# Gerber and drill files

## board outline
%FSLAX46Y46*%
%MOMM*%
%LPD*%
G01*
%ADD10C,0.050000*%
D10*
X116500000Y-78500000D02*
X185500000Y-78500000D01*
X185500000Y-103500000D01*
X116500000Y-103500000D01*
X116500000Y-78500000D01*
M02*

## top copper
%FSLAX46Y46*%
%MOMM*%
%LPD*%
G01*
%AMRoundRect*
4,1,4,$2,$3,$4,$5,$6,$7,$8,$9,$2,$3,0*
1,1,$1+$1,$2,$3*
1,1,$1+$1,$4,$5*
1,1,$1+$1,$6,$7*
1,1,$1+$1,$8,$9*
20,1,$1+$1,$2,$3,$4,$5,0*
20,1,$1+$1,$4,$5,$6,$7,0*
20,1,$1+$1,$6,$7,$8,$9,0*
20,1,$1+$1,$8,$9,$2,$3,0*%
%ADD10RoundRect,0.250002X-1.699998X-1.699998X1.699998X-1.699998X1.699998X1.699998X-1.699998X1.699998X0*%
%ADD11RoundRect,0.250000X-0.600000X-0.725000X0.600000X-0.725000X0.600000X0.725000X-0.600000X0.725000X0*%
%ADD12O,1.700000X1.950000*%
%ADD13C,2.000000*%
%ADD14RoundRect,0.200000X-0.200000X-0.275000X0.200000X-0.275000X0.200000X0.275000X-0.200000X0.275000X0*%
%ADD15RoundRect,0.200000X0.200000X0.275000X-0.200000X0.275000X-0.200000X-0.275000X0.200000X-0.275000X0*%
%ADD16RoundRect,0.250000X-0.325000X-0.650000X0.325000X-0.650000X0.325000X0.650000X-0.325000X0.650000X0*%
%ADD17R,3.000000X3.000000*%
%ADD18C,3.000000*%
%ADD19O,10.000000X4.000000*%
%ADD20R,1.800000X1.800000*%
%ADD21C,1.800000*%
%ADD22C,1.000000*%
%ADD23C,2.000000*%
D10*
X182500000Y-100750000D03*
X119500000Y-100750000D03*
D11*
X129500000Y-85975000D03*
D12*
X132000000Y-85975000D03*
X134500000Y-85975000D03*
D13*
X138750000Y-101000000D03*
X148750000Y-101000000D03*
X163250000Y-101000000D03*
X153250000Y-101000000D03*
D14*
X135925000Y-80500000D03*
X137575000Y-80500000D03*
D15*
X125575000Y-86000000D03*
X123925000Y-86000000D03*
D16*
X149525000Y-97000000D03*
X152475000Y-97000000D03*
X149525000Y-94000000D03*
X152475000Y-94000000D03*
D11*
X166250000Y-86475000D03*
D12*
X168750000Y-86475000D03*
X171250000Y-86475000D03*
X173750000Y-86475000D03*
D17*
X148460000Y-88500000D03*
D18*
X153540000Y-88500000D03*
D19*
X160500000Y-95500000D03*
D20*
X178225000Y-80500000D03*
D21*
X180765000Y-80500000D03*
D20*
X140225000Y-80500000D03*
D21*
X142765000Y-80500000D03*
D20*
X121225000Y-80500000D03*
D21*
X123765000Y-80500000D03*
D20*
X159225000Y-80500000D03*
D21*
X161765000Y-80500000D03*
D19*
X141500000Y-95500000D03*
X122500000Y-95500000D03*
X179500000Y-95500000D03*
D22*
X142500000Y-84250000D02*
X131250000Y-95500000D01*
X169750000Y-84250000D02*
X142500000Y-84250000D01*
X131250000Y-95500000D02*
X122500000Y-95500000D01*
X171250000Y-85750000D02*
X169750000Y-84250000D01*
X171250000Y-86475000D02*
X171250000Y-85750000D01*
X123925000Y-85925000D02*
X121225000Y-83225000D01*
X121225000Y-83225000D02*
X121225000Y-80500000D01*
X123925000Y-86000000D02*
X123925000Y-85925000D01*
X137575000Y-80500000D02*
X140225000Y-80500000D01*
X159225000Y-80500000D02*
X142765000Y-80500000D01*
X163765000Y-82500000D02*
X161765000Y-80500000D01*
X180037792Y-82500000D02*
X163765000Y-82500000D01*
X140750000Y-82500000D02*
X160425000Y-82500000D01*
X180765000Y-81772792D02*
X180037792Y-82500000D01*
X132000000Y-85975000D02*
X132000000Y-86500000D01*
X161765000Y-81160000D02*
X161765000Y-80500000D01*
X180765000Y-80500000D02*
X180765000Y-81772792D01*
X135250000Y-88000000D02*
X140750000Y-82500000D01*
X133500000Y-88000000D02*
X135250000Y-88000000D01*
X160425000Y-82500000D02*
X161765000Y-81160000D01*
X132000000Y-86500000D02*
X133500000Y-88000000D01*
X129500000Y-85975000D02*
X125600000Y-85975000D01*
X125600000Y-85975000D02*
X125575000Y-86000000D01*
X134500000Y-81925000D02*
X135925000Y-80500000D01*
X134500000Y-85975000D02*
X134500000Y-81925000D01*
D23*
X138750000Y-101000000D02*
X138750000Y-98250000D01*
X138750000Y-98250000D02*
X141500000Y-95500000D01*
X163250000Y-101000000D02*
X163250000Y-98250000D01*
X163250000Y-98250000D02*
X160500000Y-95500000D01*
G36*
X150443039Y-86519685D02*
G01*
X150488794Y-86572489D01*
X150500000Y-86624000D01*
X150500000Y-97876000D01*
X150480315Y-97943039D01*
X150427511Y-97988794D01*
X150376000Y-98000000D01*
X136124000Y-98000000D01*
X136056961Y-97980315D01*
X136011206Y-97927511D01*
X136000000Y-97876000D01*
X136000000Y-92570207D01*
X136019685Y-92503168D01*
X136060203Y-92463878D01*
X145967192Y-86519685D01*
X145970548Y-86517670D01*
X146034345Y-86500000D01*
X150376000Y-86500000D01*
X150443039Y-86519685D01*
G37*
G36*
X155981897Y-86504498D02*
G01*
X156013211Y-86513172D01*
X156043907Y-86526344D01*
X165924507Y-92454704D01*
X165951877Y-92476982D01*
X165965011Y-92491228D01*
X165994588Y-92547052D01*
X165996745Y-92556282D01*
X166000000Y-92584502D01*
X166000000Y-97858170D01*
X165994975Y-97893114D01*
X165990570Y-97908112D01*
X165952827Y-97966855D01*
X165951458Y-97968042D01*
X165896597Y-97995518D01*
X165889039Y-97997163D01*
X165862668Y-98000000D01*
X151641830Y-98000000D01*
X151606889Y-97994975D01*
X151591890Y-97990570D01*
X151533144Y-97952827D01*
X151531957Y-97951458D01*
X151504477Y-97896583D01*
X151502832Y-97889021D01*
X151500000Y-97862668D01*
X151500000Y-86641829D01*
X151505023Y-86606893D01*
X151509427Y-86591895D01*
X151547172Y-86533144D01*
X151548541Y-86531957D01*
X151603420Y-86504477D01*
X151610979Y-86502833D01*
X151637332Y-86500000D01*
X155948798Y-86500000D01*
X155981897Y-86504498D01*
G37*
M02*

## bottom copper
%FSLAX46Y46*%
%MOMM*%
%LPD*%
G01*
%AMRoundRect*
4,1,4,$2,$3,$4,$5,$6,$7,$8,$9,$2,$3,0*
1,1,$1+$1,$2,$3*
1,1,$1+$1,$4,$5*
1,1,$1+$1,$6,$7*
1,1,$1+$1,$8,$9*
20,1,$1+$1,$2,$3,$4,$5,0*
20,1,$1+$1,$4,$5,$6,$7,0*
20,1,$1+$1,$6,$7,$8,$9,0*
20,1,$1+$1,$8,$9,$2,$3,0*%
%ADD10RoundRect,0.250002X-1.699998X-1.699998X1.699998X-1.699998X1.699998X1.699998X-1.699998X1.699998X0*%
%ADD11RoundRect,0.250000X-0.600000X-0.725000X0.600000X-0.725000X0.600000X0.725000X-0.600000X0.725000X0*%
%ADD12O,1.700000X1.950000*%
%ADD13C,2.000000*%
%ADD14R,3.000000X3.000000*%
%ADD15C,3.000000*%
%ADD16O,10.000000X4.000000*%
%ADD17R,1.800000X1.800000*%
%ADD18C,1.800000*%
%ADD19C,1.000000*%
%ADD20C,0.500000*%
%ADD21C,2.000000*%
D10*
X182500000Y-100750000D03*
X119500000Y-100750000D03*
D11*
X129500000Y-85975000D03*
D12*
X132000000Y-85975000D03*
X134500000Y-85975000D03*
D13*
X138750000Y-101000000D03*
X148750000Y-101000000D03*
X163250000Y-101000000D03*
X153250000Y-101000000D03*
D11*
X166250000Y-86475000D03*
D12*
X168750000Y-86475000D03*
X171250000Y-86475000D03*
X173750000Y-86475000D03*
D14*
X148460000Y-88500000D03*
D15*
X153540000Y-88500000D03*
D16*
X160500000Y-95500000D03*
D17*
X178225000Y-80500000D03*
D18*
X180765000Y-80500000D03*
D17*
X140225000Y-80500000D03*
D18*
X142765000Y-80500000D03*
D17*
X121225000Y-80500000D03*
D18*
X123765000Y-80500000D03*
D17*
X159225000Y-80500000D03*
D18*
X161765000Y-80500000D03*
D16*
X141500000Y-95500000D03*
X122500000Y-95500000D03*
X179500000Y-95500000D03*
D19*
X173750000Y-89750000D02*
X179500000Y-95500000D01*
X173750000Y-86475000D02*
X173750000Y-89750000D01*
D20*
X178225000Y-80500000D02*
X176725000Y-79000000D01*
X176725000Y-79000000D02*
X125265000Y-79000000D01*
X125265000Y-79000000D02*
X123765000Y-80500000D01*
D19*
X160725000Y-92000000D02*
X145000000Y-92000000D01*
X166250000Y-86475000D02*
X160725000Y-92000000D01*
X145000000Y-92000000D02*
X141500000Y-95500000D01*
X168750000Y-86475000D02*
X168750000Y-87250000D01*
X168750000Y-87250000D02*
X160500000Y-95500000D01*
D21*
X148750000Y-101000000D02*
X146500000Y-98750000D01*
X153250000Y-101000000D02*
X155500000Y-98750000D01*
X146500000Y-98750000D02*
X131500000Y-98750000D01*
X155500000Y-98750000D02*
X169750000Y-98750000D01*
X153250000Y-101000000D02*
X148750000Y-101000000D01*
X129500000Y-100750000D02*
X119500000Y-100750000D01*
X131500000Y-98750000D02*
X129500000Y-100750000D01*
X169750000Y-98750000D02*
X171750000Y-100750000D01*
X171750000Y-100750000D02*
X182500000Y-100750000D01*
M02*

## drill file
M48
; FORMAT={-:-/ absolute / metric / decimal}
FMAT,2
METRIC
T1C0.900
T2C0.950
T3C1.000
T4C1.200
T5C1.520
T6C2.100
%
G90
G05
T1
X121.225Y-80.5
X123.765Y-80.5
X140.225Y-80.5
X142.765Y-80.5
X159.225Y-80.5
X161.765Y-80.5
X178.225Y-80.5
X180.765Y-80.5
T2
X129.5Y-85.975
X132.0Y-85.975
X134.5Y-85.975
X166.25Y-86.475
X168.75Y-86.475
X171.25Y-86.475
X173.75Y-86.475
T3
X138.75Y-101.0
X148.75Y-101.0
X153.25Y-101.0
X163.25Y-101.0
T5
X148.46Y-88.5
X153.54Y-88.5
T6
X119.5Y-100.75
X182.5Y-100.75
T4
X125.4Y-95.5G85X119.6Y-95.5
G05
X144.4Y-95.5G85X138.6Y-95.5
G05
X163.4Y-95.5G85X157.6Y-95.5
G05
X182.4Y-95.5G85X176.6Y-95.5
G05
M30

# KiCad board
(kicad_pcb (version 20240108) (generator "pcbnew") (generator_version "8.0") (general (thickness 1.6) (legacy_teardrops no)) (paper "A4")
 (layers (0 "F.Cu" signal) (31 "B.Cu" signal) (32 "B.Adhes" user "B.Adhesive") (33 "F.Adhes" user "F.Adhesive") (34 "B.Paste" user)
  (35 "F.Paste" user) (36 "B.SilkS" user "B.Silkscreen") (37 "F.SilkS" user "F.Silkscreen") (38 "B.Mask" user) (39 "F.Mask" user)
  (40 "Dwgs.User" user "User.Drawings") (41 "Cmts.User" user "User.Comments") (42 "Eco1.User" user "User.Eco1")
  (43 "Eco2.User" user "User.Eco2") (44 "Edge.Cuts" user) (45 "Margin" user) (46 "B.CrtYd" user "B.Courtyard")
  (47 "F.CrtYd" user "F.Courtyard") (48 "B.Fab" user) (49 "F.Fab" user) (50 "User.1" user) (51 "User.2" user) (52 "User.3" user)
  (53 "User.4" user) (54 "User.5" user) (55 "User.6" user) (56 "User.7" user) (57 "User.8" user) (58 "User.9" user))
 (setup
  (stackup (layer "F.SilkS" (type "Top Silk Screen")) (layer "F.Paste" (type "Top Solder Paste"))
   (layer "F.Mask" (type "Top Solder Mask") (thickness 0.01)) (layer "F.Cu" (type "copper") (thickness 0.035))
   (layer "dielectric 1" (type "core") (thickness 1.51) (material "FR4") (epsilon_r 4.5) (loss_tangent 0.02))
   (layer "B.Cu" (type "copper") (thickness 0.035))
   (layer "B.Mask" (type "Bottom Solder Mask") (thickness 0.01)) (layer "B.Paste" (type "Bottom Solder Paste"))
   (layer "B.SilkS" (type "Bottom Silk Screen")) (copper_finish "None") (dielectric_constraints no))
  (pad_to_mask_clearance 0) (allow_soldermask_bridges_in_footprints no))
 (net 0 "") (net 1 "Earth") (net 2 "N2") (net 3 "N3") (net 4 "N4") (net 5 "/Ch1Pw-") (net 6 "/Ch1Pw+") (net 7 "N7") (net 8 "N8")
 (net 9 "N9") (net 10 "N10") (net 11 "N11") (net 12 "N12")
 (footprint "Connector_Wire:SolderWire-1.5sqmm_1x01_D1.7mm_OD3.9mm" (layer "F.Cu") (at 182.5 100.75)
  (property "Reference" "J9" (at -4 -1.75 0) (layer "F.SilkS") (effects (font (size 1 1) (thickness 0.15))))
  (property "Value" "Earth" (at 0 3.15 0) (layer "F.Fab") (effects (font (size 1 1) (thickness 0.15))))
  (pad "1" thru_hole roundrect (at 0 0) (size 3.9 3.9) (drill 2.1) (layers "*.Cu" "*.Mask") (remove_unused_layers no)
   (roundrect_rratio 0.064103) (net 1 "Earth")))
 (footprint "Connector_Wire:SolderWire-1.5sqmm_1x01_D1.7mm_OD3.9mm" (layer "F.Cu") (at 119.5 100.75)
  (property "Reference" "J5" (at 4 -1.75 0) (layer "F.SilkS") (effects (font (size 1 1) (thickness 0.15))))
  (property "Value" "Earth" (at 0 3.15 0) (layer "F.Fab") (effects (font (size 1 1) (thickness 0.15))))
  (pad "1" thru_hole roundrect (at 0 0) (size 3.9 3.9) (drill 2.1) (layers "*.Cu" "*.Mask") (remove_unused_layers no)
   (roundrect_rratio 0.064103) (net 1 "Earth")))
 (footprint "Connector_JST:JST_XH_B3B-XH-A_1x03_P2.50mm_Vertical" (layer "F.Cu") (at 129.5 85.975)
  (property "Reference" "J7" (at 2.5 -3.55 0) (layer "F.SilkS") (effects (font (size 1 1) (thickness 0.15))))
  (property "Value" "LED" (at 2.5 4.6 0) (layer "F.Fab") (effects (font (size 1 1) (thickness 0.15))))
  (pad "1" thru_hole roundrect (at 0 0) (size 1.7 1.95) (drill 0.95) (layers "*.Cu" "*.Mask") (remove_unused_layers no)
   (roundrect_rratio 0.147059) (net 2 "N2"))
  (pad "2" thru_hole oval (at 2.5 0) (size 1.7 1.95) (drill 0.95) (layers "*.Cu" "*.Mask") (remove_unused_layers no) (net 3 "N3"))
  (pad "3" thru_hole oval (at 5 0) (size 1.7 1.95) (drill 0.95) (layers "*.Cu" "*.Mask") (remove_unused_layers no) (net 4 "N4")))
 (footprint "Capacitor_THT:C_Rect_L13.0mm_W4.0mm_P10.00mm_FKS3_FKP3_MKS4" (layer "F.Cu") (at 138.75 101)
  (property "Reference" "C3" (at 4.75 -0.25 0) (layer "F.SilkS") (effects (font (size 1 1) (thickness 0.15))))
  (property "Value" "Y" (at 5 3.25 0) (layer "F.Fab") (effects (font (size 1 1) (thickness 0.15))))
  (pad "1" thru_hole circle (at 0 0) (size 2 2) (drill 1) (layers "*.Cu" "*.Mask") (remove_unused_layers no) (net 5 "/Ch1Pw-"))
  (pad "2" thru_hole circle (at 10 0) (size 2 2) (drill 1) (layers "*.Cu" "*.Mask") (remove_unused_layers no) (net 1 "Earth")))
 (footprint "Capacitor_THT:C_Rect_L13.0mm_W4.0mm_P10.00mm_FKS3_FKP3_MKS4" (layer "F.Cu") (at 163.25 101 180)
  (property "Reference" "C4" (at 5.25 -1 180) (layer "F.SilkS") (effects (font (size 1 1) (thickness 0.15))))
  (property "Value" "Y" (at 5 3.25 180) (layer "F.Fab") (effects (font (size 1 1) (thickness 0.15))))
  (pad "1" thru_hole circle (at 0 0 180) (size 2 2) (drill 1) (layers "*.Cu" "*.Mask") (remove_unused_layers no) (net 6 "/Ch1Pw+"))
  (pad "2" thru_hole circle (at 10 0 180) (size 2 2) (drill 1) (layers "*.Cu" "*.Mask") (remove_unused_layers no) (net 1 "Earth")))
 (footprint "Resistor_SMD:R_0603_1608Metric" (layer "F.Cu") (at 136.75 80.5)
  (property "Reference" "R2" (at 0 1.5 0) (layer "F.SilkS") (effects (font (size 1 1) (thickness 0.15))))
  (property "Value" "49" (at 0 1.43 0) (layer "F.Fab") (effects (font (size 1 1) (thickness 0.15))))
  (pad "1" smd roundrect (at -0.825 0) (size 0.8 0.95) (layers "F.Cu" "F.Paste" "F.Mask") (roundrect_rratio 0.25) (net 4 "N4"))
  (pad "2" smd roundrect (at 0.825 0) (size 0.8 0.95) (layers "F.Cu" "F.Paste" "F.Mask") (roundrect_rratio 0.25) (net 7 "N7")))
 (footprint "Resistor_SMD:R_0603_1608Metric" (layer "F.Cu") (at 124.75 86 180)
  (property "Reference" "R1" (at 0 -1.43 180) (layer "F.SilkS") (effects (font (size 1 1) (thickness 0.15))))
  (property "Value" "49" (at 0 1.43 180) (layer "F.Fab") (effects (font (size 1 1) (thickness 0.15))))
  (pad "1" smd roundrect (at -0.825 0 180) (size 0.8 0.95) (layers "F.Cu" "F.Paste" "F.Mask") (roundrect_rratio 0.25) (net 2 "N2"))
  (pad "2" smd roundrect (at 0.825 0 180) (size 0.8 0.95) (layers "F.Cu" "F.Paste" "F.Mask") (roundrect_rratio 0.25) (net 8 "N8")))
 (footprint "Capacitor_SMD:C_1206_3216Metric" (layer "F.Cu") (at 151 97)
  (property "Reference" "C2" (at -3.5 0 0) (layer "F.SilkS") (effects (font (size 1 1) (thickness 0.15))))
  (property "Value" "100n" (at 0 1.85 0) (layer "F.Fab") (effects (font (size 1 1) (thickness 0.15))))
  (pad "1" smd roundrect (at -1.475 0) (size 1.15 1.8) (layers "F.Cu" "F.Paste" "F.Mask") (roundrect_rratio 0.217391) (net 5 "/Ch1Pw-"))
  (pad "2" smd roundrect (at 1.475 0) (size 1.15 1.8) (layers "F.Cu" "F.Paste" "F.Mask") (roundrect_rratio 0.217391) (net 6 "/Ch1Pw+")))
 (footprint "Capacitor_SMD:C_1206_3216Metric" (layer "F.Cu") (at 151 94)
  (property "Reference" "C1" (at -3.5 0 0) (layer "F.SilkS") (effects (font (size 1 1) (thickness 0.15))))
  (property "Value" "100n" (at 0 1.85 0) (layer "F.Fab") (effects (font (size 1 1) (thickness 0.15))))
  (pad "1" smd roundrect (at -1.475 0) (size 1.15 1.8) (layers "F.Cu" "F.Paste" "F.Mask") (roundrect_rratio 0.217391) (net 5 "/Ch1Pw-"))
  (pad "2" smd roundrect (at 1.475 0) (size 1.15 1.8) (layers "F.Cu" "F.Paste" "F.Mask") (roundrect_rratio 0.217391) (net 6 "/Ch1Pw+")))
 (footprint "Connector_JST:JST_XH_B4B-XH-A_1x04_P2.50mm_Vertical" (layer "F.Cu") (at 166.25 86.475)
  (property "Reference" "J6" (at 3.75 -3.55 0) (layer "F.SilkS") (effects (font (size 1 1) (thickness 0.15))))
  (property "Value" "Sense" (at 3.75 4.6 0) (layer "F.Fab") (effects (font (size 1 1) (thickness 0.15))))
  (pad "1" thru_hole roundrect (at 0 0) (size 1.7 1.95) (drill 0.95) (layers "*.Cu" "*.Mask") (remove_unused_layers no)
   (roundrect_rratio 0.147059) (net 5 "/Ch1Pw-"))
  (pad "2" thru_hole oval (at 2.5 0) (size 1.7 1.95) (drill 0.95) (layers "*.Cu" "*.Mask") (remove_unused_layers no) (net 6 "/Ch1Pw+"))
  (pad "3" thru_hole oval (at 5 0) (size 1.7 1.95) (drill 0.95) (layers "*.Cu" "*.Mask") (remove_unused_layers no) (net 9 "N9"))
  (pad "4" thru_hole oval (at 7.5 0) (size 1.7 1.95) (drill 0.95) (layers "*.Cu" "*.Mask") (remove_unused_layers no) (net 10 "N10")))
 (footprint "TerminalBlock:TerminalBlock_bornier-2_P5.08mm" (layer "F.Cu") (at 148.46 88.5)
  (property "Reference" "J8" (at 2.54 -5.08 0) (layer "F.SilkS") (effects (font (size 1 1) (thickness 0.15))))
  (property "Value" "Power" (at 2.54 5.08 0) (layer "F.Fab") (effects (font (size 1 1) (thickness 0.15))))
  (pad "1" thru_hole rect (at 0 0) (size 3 3) (drill 1.52) (layers "*.Cu" "*.Mask") (remove_unused_layers no) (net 5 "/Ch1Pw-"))
  (pad "2" thru_hole circle (at 5.08 0) (size 3 3) (drill 1.52) (layers "*.Cu" "*.Mask") (remove_unused_layers no) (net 6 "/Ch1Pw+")))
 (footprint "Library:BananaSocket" (layer "B.Cu") (at 160.5 95.5 180)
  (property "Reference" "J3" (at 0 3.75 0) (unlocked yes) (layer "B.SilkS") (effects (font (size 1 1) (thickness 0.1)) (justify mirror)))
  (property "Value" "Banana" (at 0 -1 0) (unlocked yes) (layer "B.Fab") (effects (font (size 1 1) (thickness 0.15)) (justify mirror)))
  (pad "1" thru_hole oval (at 0 0 180) (size 10 4) (drill oval 7 1.2) (layers "*.Cu" "*.Mask") (remove_unused_layers no) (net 6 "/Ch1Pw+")))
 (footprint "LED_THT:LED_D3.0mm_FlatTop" (layer "B.Cu") (at 178.225 80.5)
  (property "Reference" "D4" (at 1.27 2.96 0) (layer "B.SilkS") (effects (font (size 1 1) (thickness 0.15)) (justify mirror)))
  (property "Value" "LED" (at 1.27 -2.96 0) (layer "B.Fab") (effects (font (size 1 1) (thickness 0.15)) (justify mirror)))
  (pad "1" thru_hole rect (at 0 0) (size 1.8 1.8) (drill 0.9) (layers "*.Cu" "*.Mask") (remove_unused_layers no) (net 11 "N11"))
  (pad "2" thru_hole circle (at 2.54 0) (size 1.8 1.8) (drill 0.9) (layers "*.Cu" "*.Mask") (remove_unused_layers no) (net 3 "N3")))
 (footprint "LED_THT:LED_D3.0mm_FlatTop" (layer "B.Cu") (at 140.225 80.5)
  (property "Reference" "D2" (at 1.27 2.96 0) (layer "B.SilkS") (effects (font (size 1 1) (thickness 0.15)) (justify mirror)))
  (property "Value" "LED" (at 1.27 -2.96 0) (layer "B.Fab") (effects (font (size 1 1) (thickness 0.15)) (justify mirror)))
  (pad "1" thru_hole rect (at 0 0) (size 1.8 1.8) (drill 0.9) (layers "*.Cu" "*.Mask") (remove_unused_layers no) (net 7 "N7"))
  (pad "2" thru_hole circle (at 2.54 0) (size 1.8 1.8) (drill 0.9) (layers "*.Cu" "*.Mask") (remove_unused_layers no) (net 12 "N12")))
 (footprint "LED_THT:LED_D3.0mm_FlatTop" (layer "B.Cu") (at 121.225 80.5)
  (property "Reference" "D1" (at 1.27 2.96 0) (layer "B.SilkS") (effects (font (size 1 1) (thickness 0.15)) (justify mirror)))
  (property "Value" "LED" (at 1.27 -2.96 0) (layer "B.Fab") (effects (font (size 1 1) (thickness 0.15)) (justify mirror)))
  (pad "1" thru_hole rect (at 0 0) (size 1.8 1.8) (drill 0.9) (layers "*.Cu" "*.Mask") (remove_unused_layers no) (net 8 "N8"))
  (pad "2" thru_hole circle (at 2.54 0) (size 1.8 1.8) (drill 0.9) (layers "*.Cu" "*.Mask") (remove_unused_layers no) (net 11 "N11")))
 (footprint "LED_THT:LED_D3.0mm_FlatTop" (layer "B.Cu") (at 159.225 80.5)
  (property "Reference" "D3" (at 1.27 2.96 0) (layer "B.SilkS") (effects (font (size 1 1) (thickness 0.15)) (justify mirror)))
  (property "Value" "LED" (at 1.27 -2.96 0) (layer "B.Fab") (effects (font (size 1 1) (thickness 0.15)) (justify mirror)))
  (pad "1" thru_hole rect (at 0 0) (size 1.8 1.8) (drill 0.9) (layers "*.Cu" "*.Mask") (remove_unused_layers no) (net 12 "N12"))
  (pad "2" thru_hole circle (at 2.54 0) (size 1.8 1.8) (drill 0.9) (layers "*.Cu" "*.Mask") (remove_unused_layers no) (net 3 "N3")))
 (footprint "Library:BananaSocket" (layer "B.Cu") (at 141.5 95.5 180)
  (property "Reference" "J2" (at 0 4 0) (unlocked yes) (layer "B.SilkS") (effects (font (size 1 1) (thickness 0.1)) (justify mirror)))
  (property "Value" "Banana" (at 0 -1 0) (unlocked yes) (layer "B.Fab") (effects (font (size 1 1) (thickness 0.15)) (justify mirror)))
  (pad "1" thru_hole oval (at 0 0 180) (size 10 4) (drill oval 7 1.2) (layers "*.Cu" "*.Mask") (remove_unused_layers no) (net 5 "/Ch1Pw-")))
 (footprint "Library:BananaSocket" (layer "B.Cu") (at 122.5 95.5 180)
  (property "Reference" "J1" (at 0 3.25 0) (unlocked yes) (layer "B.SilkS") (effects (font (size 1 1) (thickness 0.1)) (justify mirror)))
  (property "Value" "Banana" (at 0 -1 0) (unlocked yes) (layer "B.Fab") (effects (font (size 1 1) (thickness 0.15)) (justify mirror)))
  (pad "1" thru_hole oval (at 0 0 180) (size 10 4) (drill oval 7 1.2) (layers "*.Cu" "*.Mask") (remove_unused_layers no) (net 9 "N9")))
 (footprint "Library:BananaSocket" (layer "B.Cu") (at 179.5 95.5 180)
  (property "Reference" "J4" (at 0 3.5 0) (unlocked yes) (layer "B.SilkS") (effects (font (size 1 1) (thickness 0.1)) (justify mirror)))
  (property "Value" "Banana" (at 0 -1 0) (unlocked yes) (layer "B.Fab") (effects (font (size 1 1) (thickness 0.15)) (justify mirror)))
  (pad "1" thru_hole oval (at 0 0 180) (size 10 4) (drill oval 7 1.2) (layers "*.Cu" "*.Mask") (remove_unused_layers no) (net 10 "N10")))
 (gr_rect (start 116.5 78.5) (end 185.5 103.5) (stroke (width 0.05) (type default)) (fill none) (layer "Edge.Cuts"))
 (segment (start 142.5 84.25) (end 131.25 95.5) (width 1) (layer "F.Cu") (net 9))
 (segment (start 169.75 84.25) (end 142.5 84.25) (width 1) (layer "F.Cu") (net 9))
 (segment (start 131.25 95.5) (end 122.5 95.5) (width 1) (layer "F.Cu") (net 9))
 (segment (start 171.25 85.75) (end 169.75 84.25) (width 1) (layer "F.Cu") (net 9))
 (segment (start 171.25 86.475) (end 171.25 85.75) (width 1) (layer "F.Cu") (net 9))
 (segment (start 173.75 89.75) (end 179.5 95.5) (width 1) (layer "B.Cu") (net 10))
 (segment (start 173.75 86.475) (end 173.75 89.75) (width 1) (layer "B.Cu") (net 10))
 (segment (start 178.225 80.5) (end 176.725 79) (width 0.5) (layer "B.Cu") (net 11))
 (segment (start 176.725 79) (end 125.265 79) (width 0.5) (layer "B.Cu") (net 11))
 (segment (start 125.265 79) (end 123.765 80.5) (width 0.5) (layer "B.Cu") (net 11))
 (segment (start 123.925 85.925) (end 121.225 83.225) (width 1) (layer "F.Cu") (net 8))
 (segment (start 121.225 83.225) (end 121.225 80.5) (width 1) (layer "F.Cu") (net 8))
 (segment (start 123.925 86) (end 123.925 85.925) (width 1) (layer "F.Cu") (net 8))
 (segment (start 137.575 80.5) (end 140.225 80.5) (width 1) (layer "F.Cu") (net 7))
 (segment (start 159.225 80.5) (end 142.765 80.5) (width 1) (layer "F.Cu") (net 12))
 (segment (start 163.765 82.5) (end 161.765 80.5) (width 1) (layer "F.Cu") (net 3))
 (segment (start 180.037792 82.5) (end 163.765 82.5) (width 1) (layer "F.Cu") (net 3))
 (segment (start 140.75 82.5) (end 160.425 82.5) (width 1) (layer "F.Cu") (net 3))
 (segment (start 180.765 81.772792) (end 180.037792 82.5) (width 1) (layer "F.Cu") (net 3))
 (segment (start 132 85.975) (end 132 86.5) (width 1) (layer "F.Cu") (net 3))
 (segment (start 161.765 81.16) (end 161.765 80.5) (width 1) (layer "F.Cu") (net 3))
 (segment (start 180.765 80.5) (end 180.765 81.772792) (width 1) (layer "F.Cu") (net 3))
 (segment (start 135.25 88) (end 140.75 82.5) (width 1) (layer "F.Cu") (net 3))
 (segment (start 133.5 88) (end 135.25 88) (width 1) (layer "F.Cu") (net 3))
 (segment (start 160.425 82.5) (end 161.765 81.16) (width 1) (layer "F.Cu") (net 3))
 (segment (start 132 86.5) (end 133.5 88) (width 1) (layer "F.Cu") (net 3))
 (segment (start 129.5 85.975) (end 125.6 85.975) (width 1) (layer "F.Cu") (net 2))
 (segment (start 125.6 85.975) (end 125.575 86) (width 1) (layer "F.Cu") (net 2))
 (segment (start 134.5 81.925) (end 135.925 80.5) (width 1) (layer "F.Cu") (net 4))
 (segment (start 134.5 85.975) (end 134.5 81.925) (width 1) (layer "F.Cu") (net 4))
 (segment (start 138.75 101) (end 138.75 98.25) (width 2) (layer "F.Cu") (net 5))
 (segment (start 138.75 98.25) (end 141.5 95.5) (width 2) (layer "F.Cu") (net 5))
 (segment (start 160.725 92) (end 145 92) (width 1) (layer "B.Cu") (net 5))
 (segment (start 166.25 86.475) (end 160.725 92) (width 1) (layer "B.Cu") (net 5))
 (segment (start 145 92) (end 141.5 95.5) (width 1) (layer "B.Cu") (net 5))
 (segment (start 163.25 101) (end 163.25 98.25) (width 2) (layer "F.Cu") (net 6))
 (segment (start 163.25 98.25) (end 160.5 95.5) (width 2) (layer "F.Cu") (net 6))
 (segment (start 168.75 86.475) (end 168.75 87.25) (width 1) (layer "B.Cu") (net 6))
 (segment (start 168.75 87.25) (end 160.5 95.5) (width 1) (layer "B.Cu") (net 6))
 (segment (start 148.75 101) (end 146.5 98.75) (width 2) (layer "B.Cu") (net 1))
 (segment (start 153.25 101) (end 155.5 98.75) (width 2) (layer "B.Cu") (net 1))
 (segment (start 146.5 98.75) (end 131.5 98.75) (width 2) (layer "B.Cu") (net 1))
 (segment (start 155.5 98.75) (end 169.75 98.75) (width 2) (layer "B.Cu") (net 1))
 (segment (start 153.25 101) (end 148.75 101) (width 2) (layer "B.Cu") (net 1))
 (segment (start 129.5 100.75) (end 119.5 100.75) (width 2) (layer "B.Cu") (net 1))
 (segment (start 131.5 98.75) (end 129.5 100.75) (width 2) (layer "B.Cu") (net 1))
 (segment (start 169.75 98.75) (end 171.75 100.75) (width 2) (layer "B.Cu") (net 1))
 (segment (start 171.75 100.75) (end 182.5 100.75) (width 2) (layer "B.Cu") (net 1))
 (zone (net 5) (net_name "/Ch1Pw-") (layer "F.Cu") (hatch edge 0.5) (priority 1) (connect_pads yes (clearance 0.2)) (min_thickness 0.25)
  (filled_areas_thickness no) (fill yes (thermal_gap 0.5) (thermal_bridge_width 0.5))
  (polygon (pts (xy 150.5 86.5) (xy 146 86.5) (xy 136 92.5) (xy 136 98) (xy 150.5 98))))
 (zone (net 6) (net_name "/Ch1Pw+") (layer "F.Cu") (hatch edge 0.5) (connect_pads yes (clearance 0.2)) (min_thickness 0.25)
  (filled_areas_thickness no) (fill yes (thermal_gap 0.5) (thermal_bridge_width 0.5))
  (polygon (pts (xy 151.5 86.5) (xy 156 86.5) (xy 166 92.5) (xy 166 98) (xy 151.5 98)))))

